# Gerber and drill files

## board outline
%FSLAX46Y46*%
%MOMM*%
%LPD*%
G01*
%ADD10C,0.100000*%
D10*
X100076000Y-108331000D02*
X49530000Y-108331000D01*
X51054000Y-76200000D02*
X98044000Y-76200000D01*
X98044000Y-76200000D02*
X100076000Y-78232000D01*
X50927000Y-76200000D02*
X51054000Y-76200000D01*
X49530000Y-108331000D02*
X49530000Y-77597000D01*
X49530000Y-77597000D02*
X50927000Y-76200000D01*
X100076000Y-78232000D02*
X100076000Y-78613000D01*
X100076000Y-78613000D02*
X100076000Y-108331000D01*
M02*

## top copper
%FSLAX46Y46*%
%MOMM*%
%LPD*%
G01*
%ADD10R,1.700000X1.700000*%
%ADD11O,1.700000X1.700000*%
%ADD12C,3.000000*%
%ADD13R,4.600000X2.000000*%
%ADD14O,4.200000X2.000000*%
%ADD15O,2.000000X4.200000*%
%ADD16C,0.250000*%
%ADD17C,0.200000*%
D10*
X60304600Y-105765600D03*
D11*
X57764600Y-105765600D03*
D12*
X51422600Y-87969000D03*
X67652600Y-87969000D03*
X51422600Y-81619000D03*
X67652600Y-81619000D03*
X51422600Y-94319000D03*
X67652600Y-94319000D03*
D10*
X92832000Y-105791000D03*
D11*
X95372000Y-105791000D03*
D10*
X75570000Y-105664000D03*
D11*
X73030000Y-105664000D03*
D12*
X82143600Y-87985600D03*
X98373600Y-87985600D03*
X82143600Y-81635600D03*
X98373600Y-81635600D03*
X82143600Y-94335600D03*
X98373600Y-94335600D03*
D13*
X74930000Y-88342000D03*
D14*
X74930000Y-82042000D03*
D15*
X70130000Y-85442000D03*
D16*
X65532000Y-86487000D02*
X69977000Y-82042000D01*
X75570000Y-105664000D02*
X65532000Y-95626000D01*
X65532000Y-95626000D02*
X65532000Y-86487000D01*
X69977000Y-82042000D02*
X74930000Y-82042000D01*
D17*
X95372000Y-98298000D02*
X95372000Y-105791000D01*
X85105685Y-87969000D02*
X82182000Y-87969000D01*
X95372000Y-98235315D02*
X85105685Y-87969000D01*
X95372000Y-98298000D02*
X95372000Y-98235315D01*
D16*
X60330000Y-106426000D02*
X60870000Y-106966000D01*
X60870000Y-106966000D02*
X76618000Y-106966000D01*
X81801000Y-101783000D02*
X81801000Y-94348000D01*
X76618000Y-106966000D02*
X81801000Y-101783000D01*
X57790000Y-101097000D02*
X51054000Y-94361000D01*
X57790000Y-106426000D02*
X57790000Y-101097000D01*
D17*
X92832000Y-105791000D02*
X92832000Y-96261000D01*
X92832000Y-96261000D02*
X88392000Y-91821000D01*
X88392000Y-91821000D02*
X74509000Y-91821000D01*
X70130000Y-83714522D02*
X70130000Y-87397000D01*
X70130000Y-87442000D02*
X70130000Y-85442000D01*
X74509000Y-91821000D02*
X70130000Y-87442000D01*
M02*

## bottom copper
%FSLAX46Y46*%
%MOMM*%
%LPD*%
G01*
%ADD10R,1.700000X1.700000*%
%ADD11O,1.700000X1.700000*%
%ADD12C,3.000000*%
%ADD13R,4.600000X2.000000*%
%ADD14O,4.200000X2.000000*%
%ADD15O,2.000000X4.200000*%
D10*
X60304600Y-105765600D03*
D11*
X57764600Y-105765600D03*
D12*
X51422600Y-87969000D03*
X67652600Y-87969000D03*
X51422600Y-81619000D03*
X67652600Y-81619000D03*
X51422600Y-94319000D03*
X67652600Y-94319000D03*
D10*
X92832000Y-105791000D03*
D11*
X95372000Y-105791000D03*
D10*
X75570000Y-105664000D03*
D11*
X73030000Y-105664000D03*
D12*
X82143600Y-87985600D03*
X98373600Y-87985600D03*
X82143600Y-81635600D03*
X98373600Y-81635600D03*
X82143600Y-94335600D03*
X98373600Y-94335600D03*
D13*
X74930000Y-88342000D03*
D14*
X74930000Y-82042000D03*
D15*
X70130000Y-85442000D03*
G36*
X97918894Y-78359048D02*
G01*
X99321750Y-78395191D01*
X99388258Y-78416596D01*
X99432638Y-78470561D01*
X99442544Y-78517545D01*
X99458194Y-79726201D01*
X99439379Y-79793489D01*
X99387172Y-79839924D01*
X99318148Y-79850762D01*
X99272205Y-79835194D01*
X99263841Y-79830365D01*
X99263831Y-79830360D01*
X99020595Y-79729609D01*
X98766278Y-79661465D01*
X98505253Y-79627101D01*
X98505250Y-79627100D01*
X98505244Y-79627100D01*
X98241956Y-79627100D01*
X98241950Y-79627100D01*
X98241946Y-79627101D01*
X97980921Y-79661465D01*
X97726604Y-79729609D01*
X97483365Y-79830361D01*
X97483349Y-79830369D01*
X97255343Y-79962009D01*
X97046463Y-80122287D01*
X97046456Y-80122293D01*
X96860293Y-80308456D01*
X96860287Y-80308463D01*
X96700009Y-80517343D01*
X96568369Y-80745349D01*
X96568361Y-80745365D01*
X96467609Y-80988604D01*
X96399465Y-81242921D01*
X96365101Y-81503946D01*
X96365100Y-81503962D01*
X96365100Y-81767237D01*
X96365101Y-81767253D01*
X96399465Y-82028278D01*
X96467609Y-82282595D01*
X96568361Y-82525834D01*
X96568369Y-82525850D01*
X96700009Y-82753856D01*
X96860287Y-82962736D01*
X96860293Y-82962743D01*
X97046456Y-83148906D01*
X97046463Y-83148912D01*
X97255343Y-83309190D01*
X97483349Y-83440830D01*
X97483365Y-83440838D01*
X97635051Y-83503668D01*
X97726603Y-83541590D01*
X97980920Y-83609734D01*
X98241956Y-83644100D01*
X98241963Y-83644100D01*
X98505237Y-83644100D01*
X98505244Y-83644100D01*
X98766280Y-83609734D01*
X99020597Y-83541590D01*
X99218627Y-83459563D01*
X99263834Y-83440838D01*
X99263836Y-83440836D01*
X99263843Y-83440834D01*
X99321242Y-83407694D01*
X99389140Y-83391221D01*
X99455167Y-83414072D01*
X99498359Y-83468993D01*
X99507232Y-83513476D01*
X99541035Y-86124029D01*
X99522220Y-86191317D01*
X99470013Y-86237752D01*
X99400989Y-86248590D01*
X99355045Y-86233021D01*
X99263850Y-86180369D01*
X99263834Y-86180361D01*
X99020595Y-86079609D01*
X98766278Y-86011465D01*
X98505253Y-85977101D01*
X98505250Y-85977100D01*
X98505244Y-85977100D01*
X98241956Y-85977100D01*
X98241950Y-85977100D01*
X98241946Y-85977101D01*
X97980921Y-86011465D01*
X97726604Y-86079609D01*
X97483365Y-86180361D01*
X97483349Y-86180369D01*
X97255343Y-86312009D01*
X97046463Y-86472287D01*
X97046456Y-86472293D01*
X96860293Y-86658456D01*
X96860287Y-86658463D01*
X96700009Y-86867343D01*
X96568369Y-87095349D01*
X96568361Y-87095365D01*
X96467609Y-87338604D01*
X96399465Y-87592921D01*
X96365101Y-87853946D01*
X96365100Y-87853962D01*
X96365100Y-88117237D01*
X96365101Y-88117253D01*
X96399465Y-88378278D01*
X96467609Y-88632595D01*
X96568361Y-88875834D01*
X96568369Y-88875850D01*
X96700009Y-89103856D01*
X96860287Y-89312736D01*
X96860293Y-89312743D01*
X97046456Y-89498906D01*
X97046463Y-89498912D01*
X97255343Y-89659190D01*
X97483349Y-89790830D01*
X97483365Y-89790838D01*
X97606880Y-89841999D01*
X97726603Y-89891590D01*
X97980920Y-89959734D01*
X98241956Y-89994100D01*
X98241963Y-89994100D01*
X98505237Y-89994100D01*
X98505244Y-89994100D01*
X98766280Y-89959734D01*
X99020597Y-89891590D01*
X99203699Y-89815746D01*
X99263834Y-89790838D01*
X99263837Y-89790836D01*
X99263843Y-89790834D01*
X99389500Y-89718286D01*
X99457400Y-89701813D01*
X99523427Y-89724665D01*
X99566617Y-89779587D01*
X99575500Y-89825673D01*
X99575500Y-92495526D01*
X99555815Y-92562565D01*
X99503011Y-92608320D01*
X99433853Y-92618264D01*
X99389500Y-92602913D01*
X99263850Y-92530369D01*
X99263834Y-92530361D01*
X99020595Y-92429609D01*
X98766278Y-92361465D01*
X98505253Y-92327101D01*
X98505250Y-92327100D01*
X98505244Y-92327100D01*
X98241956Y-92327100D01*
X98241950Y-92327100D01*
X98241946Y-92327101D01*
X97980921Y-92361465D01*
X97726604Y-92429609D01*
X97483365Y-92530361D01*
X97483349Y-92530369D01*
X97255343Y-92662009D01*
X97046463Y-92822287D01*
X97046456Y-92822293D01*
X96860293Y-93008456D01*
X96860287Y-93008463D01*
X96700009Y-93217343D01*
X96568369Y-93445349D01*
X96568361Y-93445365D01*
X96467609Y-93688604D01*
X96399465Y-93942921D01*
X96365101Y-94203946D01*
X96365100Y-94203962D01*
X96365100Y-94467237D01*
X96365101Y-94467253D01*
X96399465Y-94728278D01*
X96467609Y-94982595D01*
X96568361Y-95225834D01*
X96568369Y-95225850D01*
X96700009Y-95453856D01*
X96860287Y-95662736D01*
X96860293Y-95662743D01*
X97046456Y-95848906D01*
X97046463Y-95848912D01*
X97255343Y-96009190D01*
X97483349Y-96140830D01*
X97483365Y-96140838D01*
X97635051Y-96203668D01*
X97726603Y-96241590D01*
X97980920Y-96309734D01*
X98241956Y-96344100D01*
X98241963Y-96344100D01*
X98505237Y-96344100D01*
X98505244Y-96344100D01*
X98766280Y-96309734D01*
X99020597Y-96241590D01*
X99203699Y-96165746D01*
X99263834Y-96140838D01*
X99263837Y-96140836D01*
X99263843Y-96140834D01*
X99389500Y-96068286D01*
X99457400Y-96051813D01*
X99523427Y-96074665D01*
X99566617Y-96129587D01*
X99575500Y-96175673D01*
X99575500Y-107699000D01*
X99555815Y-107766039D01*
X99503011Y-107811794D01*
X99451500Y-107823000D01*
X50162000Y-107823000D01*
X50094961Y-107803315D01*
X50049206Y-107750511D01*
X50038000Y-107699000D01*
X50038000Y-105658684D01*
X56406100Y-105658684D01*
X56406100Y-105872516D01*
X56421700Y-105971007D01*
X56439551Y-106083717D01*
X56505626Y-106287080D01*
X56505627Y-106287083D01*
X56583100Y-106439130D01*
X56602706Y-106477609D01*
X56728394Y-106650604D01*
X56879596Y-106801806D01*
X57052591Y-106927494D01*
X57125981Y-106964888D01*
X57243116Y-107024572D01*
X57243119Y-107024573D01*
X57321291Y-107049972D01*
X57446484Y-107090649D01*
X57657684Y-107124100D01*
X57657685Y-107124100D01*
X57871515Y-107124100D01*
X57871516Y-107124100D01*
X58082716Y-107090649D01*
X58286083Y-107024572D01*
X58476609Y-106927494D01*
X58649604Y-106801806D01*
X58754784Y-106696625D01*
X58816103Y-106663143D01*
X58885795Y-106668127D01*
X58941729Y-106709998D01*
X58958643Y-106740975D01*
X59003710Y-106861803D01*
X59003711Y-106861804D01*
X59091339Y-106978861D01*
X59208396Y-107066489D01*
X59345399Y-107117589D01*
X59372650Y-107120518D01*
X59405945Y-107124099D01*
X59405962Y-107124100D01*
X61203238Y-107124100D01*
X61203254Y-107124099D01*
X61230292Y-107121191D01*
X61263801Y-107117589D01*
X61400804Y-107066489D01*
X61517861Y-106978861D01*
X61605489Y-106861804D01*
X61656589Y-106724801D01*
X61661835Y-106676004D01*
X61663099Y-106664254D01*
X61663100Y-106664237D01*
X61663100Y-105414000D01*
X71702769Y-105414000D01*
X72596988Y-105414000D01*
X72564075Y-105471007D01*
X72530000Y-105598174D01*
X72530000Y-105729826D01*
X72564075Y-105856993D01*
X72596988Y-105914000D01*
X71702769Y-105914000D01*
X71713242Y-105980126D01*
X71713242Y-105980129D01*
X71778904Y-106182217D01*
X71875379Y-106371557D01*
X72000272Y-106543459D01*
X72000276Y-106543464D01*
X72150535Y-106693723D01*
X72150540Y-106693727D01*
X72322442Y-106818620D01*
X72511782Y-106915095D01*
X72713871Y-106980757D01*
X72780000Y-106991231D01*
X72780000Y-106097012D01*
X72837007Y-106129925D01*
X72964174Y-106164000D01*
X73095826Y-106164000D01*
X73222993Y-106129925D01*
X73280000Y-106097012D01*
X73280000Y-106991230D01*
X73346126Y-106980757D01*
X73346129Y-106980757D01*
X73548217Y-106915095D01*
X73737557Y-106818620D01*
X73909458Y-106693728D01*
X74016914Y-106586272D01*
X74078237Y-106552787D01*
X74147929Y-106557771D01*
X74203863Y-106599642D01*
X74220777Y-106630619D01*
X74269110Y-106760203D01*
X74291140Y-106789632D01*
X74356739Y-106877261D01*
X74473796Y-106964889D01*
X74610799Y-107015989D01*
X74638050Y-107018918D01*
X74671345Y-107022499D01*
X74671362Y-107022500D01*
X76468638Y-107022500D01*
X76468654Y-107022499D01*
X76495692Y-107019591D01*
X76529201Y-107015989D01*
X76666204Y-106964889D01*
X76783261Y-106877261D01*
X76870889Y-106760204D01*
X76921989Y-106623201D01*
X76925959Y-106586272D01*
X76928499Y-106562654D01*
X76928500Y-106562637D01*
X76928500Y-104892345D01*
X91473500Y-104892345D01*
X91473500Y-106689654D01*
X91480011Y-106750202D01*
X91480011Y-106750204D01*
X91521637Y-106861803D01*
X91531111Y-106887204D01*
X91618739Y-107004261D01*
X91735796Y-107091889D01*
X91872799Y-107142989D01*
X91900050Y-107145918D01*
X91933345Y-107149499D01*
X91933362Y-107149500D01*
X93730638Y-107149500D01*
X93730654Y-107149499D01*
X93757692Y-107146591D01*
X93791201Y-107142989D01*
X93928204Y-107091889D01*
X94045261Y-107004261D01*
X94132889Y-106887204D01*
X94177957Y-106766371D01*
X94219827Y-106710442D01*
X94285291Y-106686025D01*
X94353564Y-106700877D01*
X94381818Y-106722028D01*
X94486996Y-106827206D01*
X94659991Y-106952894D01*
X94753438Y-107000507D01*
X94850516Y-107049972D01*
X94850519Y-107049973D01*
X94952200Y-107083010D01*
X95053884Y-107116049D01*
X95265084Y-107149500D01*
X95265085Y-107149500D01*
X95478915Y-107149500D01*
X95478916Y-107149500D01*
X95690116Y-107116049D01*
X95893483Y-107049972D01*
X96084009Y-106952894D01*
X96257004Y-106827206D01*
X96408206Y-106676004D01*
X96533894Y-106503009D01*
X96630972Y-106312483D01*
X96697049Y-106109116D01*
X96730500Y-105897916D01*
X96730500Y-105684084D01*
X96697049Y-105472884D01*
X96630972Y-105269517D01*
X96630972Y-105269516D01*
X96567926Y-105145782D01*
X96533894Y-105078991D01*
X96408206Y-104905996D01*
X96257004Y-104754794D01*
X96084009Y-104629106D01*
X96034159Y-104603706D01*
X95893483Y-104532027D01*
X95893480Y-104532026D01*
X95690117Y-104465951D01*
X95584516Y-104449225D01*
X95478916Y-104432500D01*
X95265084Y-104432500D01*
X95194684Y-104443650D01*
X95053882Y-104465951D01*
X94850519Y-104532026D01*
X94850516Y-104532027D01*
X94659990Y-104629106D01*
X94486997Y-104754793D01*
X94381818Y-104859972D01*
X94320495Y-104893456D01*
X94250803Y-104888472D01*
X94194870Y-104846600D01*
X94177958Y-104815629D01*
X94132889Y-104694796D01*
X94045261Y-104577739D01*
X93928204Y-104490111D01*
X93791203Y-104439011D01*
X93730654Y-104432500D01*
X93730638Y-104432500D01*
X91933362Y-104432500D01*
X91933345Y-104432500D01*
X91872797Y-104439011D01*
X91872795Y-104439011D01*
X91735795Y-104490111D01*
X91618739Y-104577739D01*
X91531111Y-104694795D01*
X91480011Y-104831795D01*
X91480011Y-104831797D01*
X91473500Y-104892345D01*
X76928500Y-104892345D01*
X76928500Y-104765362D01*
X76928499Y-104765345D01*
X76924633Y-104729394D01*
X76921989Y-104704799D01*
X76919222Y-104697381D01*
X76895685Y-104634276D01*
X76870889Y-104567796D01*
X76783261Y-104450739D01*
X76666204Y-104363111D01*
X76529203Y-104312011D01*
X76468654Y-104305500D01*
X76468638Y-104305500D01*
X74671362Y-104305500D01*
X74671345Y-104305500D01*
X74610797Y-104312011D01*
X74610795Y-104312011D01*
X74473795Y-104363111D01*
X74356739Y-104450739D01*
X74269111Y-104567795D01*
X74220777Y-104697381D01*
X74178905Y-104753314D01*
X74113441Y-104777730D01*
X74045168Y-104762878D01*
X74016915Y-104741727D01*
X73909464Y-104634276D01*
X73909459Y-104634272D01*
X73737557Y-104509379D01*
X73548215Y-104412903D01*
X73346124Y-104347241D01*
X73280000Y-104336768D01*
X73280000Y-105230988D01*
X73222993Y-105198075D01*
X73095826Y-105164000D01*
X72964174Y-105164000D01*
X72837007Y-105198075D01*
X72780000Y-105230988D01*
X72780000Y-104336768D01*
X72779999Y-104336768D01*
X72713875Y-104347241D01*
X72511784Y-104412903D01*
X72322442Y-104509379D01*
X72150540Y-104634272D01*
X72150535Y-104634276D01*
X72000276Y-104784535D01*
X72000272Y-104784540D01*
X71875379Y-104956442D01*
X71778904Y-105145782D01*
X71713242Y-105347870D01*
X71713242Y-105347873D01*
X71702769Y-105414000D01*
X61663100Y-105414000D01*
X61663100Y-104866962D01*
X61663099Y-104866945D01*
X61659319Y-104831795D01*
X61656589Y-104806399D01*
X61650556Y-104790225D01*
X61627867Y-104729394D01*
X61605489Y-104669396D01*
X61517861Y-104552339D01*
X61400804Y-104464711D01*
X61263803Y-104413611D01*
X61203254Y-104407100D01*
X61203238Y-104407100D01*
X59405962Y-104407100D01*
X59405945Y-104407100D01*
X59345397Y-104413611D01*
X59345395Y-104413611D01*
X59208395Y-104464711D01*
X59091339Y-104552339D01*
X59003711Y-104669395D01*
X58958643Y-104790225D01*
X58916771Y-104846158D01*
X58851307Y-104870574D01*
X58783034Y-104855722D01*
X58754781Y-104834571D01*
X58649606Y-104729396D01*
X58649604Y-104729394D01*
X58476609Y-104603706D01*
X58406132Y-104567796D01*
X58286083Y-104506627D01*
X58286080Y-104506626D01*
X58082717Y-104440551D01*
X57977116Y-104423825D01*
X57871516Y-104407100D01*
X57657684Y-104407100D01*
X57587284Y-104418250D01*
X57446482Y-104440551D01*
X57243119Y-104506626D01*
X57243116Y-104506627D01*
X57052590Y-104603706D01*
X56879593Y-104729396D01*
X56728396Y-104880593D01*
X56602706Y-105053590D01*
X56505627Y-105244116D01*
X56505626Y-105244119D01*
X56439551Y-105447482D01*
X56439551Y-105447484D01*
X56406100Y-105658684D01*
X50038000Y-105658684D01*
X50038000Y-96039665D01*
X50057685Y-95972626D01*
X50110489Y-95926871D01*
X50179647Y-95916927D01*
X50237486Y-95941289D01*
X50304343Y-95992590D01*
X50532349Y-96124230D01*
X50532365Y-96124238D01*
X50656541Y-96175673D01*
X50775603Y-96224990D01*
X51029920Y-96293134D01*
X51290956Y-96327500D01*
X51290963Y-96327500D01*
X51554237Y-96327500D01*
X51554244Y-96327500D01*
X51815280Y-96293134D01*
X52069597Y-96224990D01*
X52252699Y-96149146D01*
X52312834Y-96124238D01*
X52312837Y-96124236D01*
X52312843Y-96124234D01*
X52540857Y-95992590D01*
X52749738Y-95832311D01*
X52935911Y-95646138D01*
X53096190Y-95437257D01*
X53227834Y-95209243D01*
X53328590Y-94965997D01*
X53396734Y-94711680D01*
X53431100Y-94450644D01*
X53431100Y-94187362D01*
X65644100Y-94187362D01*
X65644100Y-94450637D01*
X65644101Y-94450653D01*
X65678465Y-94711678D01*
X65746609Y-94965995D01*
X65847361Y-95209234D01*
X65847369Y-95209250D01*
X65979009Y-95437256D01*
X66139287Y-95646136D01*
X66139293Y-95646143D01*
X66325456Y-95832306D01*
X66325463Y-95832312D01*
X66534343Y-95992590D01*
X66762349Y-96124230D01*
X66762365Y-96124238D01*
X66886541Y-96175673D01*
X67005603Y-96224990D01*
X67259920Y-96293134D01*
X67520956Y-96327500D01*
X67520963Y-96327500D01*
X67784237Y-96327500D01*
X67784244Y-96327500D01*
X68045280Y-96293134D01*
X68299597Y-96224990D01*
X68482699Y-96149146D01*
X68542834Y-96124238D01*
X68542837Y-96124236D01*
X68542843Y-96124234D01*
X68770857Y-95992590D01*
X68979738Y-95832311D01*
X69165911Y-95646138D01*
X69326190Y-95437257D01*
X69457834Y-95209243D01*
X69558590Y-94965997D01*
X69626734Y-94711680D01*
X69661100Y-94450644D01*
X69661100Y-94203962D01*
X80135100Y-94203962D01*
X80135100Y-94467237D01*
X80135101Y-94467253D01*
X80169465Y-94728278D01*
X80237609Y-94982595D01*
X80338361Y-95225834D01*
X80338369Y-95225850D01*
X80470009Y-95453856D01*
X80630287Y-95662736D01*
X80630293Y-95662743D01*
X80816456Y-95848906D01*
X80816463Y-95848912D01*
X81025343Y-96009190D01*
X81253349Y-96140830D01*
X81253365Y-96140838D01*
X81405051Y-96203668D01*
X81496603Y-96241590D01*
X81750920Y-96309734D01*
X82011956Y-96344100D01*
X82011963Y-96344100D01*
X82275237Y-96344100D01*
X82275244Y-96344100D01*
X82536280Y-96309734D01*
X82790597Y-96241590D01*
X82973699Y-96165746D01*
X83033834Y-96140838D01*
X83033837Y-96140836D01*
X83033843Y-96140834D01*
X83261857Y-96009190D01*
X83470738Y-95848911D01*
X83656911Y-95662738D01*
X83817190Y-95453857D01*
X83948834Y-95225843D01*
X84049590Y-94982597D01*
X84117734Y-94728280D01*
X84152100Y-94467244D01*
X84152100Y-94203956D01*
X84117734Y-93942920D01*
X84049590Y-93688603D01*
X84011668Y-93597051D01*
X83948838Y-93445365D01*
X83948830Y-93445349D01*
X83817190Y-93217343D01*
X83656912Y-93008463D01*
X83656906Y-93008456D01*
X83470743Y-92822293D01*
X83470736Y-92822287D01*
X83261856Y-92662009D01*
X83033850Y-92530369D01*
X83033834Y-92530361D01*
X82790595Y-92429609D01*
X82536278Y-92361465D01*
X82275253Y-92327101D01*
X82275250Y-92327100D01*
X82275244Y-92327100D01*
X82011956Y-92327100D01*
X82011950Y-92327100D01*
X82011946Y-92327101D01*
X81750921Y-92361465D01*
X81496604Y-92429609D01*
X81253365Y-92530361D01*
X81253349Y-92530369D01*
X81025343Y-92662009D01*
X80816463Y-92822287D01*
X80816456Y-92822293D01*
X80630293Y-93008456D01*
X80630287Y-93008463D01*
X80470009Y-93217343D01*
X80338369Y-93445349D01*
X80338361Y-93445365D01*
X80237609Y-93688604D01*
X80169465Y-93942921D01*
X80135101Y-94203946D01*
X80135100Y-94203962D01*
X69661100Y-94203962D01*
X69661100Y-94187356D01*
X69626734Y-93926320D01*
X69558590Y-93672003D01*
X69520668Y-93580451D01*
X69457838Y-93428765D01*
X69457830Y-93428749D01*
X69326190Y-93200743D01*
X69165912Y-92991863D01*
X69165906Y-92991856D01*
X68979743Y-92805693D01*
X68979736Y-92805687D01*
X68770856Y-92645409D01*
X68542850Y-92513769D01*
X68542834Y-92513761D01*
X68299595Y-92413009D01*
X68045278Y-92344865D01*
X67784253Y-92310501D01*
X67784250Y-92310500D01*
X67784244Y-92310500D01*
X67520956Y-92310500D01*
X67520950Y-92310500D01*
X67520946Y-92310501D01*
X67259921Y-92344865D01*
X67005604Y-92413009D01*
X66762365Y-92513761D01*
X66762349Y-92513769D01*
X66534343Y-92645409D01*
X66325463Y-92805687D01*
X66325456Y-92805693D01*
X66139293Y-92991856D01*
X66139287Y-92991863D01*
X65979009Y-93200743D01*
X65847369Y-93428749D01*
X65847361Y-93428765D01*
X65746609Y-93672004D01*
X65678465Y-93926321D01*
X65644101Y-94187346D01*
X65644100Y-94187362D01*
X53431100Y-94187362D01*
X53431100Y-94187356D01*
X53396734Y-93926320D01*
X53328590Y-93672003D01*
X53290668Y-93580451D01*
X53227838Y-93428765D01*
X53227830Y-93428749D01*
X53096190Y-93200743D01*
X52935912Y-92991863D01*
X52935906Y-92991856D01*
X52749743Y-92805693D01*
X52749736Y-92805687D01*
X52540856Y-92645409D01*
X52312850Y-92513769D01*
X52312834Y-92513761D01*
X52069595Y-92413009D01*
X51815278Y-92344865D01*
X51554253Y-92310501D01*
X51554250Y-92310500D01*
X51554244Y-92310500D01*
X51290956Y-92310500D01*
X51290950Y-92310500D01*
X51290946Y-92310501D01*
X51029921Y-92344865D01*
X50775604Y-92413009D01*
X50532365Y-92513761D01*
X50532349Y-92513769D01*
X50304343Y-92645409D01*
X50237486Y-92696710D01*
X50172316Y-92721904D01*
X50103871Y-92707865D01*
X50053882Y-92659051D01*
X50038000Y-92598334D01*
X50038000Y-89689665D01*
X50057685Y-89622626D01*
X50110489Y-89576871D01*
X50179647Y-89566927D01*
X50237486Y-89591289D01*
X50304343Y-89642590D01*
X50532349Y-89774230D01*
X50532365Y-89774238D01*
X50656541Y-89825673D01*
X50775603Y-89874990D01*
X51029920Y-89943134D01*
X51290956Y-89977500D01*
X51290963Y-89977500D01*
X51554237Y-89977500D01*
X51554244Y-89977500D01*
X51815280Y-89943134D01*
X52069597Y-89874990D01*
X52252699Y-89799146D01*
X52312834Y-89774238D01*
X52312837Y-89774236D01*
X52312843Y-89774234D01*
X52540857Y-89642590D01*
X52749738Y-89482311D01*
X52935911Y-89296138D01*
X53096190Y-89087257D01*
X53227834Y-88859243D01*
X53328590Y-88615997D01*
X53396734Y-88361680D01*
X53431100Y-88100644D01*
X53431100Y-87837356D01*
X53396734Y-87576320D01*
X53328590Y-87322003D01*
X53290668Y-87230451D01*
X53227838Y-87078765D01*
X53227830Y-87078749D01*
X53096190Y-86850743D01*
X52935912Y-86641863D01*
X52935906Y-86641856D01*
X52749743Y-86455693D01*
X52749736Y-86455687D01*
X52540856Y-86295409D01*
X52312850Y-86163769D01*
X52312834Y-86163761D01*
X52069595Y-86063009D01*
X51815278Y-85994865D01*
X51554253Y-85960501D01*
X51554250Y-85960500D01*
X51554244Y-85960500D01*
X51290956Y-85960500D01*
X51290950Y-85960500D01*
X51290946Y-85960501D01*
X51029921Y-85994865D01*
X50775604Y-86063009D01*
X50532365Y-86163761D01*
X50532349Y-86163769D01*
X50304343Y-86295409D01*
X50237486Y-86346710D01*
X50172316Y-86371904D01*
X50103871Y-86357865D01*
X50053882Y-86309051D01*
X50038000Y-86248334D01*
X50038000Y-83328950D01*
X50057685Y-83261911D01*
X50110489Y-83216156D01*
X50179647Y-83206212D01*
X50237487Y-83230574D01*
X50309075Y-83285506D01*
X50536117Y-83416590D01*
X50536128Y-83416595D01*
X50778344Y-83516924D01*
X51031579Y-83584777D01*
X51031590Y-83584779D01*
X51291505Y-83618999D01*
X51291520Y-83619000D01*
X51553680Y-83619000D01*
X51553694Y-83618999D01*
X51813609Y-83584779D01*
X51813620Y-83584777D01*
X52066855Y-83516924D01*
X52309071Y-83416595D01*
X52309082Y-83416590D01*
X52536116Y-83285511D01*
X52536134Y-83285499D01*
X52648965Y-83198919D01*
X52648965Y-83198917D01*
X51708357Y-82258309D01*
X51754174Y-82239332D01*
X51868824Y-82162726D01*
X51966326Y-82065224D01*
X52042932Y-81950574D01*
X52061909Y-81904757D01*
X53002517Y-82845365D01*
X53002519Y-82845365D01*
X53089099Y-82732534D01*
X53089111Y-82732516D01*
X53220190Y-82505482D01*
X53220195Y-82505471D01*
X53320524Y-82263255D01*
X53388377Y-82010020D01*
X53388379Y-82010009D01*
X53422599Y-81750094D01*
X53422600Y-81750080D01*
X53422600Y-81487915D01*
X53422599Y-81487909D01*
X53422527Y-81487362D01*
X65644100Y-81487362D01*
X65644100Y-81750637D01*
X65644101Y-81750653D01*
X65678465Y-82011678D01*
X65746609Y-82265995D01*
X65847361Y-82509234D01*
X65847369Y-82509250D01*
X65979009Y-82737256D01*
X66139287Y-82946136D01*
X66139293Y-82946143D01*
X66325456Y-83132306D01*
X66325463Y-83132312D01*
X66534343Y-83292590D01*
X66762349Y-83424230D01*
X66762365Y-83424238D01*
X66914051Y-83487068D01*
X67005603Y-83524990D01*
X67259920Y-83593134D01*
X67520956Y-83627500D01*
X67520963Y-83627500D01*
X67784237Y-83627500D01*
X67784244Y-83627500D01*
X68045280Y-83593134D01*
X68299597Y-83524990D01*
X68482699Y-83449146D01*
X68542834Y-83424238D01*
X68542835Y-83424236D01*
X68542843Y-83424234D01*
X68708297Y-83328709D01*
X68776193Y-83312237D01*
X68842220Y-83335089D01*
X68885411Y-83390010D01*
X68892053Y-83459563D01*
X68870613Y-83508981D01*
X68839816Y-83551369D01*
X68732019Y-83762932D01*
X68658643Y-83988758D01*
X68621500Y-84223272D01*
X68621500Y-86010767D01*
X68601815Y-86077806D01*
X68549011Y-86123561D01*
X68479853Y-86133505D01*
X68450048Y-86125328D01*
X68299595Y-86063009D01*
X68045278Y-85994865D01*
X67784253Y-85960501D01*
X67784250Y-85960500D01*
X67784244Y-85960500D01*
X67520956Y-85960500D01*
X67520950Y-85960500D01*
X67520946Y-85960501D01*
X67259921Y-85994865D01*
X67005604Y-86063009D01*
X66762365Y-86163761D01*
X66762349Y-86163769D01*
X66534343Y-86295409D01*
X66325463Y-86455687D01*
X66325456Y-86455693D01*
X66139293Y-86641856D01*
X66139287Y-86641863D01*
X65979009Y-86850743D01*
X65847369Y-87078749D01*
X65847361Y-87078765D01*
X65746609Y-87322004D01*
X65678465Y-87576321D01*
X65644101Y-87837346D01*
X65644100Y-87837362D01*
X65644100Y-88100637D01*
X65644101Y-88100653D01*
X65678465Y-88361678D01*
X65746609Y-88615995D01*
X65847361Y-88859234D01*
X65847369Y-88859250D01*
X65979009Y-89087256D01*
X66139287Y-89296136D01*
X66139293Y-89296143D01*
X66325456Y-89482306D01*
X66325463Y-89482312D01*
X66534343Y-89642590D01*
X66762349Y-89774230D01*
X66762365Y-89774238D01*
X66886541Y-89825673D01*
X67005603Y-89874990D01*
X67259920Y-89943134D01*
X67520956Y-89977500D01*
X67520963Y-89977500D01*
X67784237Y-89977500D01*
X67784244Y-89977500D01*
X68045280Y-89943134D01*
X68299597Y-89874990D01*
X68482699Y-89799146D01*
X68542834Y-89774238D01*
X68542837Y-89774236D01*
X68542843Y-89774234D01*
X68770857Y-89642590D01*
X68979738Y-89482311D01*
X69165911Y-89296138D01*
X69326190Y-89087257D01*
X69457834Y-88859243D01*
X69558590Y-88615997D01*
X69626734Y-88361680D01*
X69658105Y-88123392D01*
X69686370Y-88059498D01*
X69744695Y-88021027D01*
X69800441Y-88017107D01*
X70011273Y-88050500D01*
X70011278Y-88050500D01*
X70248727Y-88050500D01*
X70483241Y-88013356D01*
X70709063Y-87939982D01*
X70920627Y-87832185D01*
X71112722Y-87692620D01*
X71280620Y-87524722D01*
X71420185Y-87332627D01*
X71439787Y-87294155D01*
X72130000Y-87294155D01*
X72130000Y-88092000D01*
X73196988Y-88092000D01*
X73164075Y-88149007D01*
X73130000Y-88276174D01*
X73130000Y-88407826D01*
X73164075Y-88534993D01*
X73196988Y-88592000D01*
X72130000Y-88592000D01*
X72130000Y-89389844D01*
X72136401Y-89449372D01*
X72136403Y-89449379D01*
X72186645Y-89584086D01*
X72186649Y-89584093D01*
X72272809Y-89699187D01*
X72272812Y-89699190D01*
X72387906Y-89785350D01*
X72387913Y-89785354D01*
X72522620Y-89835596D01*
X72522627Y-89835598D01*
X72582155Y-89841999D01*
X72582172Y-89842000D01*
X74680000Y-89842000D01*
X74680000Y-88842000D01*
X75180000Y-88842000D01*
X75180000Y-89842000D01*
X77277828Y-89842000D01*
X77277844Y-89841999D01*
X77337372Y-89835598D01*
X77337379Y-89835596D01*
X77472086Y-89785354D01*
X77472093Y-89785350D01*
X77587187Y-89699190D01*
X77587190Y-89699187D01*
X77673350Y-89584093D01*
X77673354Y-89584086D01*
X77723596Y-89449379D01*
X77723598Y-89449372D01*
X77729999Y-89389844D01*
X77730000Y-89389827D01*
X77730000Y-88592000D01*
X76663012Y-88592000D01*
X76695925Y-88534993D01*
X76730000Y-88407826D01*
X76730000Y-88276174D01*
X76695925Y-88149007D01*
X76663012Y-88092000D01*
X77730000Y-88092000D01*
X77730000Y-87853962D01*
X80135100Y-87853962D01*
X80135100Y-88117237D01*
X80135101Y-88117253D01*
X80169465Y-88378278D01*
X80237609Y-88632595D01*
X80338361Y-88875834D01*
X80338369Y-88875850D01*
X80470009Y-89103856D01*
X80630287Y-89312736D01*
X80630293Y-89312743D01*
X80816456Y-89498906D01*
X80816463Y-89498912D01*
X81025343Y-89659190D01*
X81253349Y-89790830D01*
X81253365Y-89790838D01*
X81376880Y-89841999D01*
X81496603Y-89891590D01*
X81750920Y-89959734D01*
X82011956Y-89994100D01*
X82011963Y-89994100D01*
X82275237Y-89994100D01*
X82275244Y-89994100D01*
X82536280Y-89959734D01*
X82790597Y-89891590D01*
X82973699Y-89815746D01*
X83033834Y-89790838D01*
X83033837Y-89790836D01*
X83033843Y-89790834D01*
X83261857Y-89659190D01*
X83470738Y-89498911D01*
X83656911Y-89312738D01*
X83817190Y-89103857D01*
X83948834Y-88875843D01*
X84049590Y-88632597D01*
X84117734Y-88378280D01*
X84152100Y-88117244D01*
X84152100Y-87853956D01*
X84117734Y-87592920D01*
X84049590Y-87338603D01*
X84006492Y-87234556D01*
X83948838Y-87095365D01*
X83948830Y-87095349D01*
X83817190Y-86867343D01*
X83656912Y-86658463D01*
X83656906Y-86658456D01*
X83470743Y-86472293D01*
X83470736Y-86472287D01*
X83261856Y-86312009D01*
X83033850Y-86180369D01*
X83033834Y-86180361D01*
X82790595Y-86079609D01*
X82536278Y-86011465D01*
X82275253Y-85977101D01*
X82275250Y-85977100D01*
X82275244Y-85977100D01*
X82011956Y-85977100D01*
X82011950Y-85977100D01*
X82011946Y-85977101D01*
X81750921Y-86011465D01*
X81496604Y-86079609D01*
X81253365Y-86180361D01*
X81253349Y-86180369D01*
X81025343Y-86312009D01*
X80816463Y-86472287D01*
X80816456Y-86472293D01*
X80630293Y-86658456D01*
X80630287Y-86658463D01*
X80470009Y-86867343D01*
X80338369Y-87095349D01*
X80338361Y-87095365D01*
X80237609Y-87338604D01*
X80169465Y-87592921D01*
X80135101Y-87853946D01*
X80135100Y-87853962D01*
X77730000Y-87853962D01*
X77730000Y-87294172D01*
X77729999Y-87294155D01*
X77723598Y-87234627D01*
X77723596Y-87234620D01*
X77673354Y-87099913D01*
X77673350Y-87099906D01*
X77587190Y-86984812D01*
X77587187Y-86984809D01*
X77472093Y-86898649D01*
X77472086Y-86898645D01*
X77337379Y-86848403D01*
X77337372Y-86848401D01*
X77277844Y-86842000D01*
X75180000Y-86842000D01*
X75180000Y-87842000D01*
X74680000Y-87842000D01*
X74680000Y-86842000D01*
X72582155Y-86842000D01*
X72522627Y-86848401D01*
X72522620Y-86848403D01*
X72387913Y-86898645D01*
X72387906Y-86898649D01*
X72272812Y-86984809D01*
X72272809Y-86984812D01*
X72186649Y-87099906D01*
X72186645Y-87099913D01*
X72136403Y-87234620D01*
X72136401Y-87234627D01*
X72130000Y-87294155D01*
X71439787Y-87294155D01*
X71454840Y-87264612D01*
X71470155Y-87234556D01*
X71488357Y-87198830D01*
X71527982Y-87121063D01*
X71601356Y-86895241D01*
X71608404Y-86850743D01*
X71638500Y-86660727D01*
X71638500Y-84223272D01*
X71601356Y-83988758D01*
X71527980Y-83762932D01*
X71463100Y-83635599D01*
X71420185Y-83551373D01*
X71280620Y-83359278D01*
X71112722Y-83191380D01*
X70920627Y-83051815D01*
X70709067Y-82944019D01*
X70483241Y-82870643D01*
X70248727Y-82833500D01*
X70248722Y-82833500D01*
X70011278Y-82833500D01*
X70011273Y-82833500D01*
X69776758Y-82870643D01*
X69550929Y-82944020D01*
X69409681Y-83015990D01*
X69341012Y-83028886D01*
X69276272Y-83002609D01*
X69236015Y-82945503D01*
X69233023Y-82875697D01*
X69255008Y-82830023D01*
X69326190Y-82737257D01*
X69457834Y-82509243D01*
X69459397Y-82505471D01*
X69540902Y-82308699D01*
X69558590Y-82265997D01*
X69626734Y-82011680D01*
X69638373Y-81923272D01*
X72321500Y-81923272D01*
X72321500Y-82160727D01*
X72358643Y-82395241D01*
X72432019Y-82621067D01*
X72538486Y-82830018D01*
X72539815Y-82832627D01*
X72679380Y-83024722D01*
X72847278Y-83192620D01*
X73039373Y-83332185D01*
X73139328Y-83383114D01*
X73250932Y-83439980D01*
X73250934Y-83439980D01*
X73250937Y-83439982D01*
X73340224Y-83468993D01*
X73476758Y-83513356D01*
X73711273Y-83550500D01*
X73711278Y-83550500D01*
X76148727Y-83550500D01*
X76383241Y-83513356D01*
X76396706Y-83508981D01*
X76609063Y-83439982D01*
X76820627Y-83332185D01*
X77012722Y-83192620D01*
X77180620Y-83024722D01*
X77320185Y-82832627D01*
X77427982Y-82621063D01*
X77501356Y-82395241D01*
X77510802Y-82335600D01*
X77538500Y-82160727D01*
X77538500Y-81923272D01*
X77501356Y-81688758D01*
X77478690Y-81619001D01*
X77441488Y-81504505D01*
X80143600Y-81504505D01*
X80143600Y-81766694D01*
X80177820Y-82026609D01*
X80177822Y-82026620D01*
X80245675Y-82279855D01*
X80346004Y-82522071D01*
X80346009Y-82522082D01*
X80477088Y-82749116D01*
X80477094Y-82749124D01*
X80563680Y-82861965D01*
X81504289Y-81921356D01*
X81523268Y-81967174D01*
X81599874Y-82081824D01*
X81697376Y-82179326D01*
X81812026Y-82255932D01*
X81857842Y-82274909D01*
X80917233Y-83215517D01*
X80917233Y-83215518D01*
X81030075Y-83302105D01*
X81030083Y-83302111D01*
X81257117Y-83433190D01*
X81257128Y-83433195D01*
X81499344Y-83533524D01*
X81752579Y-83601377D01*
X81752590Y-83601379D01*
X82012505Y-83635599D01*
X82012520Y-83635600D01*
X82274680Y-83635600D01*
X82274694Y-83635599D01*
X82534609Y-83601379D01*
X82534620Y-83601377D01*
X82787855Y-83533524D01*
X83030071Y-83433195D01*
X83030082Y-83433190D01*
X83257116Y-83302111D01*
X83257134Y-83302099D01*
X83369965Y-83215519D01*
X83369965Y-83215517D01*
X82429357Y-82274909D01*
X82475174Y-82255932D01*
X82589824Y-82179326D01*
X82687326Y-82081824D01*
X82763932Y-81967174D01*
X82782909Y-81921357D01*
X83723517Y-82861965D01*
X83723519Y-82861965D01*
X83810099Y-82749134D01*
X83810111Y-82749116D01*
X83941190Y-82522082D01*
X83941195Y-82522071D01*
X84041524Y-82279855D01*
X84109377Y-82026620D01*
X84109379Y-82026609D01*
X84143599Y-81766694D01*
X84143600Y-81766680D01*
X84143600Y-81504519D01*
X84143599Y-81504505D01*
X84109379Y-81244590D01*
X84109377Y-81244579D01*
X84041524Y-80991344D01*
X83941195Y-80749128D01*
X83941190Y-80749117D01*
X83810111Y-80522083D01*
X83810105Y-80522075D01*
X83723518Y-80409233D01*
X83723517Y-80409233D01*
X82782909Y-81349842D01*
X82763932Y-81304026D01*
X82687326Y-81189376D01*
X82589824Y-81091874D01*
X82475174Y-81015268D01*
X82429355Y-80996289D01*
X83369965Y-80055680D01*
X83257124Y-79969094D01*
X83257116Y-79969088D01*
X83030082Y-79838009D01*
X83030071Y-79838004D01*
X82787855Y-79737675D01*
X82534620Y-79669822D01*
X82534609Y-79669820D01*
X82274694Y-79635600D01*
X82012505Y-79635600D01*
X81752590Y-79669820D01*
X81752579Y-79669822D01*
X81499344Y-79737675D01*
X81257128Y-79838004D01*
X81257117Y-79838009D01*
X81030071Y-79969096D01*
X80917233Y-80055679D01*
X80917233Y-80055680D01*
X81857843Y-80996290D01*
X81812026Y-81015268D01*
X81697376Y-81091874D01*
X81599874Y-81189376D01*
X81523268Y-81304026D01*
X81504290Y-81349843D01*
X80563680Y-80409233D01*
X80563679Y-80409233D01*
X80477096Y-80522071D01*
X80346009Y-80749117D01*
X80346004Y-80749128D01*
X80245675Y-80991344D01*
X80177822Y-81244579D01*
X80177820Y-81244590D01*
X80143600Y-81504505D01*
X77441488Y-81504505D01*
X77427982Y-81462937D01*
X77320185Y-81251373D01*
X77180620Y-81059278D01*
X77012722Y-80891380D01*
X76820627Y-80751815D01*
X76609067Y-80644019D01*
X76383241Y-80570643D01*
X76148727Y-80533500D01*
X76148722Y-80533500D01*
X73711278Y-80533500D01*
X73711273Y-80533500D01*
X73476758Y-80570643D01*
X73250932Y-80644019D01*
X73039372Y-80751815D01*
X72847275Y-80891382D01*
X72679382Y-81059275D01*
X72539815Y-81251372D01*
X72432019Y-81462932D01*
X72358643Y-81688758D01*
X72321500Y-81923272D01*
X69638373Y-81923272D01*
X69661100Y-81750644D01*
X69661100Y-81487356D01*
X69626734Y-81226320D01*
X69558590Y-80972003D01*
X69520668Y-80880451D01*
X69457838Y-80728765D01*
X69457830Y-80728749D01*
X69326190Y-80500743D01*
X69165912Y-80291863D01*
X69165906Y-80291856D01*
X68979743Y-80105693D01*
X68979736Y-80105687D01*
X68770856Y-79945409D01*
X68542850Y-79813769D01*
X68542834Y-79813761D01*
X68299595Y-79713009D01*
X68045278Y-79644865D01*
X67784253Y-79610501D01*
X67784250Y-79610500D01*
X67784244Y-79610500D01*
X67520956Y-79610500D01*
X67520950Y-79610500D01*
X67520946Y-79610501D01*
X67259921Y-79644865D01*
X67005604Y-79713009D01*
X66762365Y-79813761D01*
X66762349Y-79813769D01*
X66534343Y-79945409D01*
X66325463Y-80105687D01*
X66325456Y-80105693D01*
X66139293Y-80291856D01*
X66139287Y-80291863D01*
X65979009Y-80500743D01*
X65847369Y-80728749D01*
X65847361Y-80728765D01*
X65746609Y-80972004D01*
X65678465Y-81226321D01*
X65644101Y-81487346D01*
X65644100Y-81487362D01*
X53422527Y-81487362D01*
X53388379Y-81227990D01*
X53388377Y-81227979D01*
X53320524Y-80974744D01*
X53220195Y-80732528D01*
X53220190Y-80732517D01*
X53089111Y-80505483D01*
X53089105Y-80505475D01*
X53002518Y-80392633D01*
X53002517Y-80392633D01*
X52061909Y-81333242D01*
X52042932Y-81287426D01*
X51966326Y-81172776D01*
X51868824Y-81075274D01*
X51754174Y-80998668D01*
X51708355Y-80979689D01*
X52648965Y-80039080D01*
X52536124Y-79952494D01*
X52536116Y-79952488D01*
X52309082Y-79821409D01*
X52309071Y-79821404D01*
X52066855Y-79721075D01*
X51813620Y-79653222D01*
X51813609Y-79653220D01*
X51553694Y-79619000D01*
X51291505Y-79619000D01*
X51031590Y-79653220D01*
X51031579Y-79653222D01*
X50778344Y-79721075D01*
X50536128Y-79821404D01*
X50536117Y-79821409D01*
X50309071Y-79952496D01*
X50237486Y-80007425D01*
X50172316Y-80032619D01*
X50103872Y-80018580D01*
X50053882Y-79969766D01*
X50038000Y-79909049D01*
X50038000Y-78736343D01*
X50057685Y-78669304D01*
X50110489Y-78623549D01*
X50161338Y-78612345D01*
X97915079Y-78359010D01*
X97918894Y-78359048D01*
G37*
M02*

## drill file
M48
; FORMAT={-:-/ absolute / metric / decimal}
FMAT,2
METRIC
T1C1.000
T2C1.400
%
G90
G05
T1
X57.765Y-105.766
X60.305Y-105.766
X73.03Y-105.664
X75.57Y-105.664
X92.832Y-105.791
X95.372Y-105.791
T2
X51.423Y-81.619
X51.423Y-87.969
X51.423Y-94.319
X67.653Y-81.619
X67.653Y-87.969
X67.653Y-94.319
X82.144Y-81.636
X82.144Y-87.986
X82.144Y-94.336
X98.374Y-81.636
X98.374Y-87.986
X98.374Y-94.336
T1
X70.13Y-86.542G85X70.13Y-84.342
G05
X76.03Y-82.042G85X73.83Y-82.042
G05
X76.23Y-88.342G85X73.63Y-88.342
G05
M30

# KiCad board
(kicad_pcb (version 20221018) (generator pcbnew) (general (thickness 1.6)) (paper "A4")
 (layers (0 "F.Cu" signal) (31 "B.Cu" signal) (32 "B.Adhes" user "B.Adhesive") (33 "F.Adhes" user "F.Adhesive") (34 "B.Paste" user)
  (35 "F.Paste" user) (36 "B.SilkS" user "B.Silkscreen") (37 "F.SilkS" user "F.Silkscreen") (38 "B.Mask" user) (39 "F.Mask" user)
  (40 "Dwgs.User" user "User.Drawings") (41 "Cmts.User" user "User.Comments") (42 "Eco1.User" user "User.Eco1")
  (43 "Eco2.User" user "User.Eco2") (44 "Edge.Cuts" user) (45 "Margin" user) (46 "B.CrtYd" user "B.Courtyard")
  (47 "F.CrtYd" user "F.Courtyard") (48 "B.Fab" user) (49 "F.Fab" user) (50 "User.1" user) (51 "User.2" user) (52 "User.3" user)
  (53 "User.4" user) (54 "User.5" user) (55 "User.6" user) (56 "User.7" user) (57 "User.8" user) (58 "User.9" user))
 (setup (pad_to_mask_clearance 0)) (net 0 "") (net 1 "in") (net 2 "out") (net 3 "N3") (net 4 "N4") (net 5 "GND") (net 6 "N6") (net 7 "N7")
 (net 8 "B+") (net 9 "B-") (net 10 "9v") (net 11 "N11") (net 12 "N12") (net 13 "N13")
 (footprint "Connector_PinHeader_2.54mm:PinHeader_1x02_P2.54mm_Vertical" (layer "F.Cu") (at 60.3046 105.7656 -90)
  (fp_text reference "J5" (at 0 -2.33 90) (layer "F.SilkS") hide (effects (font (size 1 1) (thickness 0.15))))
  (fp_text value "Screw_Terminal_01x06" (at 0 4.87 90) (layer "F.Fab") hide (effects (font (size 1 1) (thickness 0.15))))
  (pad "1" thru_hole rect (at 0 0 270) (size 1.7 1.7) (drill 1) (layers "*.Cu" "*.Mask") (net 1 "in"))
  (pad "2" thru_hole oval (at 0 2.54 270) (size 1.7 1.7) (drill 1) (layers "*.Cu" "*.Mask") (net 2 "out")))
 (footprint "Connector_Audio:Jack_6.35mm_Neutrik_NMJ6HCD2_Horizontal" (layer "F.Cu") (at 51.4226 94.319 90)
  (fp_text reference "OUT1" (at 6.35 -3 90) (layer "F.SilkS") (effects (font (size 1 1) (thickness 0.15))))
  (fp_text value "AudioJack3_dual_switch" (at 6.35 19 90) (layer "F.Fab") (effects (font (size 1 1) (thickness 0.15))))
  (pad "R" thru_hole circle (at 6.35 0 90) (size 3 3) (drill 1.4) (layers "*.Cu" "*.Mask") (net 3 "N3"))
  (pad "RN" thru_hole circle (at 6.35 16.23 90) (size 3 3) (drill 1.4) (layers "*.Cu" "*.Mask") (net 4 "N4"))
  (pad "S" thru_hole circle (at 12.7 0 90) (size 3 3) (drill 1.4) (layers "*.Cu" "*.Mask") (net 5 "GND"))
  (pad "SN" thru_hole circle (at 12.7 16.23 90) (size 3 3) (drill 1.4) (layers "*.Cu" "*.Mask") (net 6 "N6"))
  (pad "T" thru_hole circle (at 0 0 90) (size 3 3) (drill 1.4) (layers "*.Cu" "*.Mask") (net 2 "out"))
  (pad "TN" thru_hole circle (at 0 16.23 90) (size 3 3) (drill 1.4) (layers "*.Cu" "*.Mask") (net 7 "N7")))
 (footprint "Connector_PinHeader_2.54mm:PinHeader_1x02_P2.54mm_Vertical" (layer "F.Cu") (at 92.832 105.791 90)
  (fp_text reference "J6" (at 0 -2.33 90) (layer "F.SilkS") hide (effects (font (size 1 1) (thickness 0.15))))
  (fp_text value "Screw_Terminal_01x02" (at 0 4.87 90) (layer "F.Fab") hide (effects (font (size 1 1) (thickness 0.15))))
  (pad "1" thru_hole rect (at 0 0 90) (size 1.7 1.7) (drill 1) (layers "*.Cu" "*.Mask") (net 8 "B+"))
  (pad "2" thru_hole oval (at 0 2.54 90) (size 1.7 1.7) (drill 1) (layers "*.Cu" "*.Mask") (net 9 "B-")))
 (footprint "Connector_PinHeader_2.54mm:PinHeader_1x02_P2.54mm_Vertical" (layer "F.Cu") (at 75.57 105.664 -90)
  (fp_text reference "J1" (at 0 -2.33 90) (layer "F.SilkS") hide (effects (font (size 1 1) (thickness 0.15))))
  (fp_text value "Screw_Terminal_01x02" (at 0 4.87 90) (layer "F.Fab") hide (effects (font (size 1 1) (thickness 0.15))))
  (pad "1" thru_hole rect (at 0 0 270) (size 1.7 1.7) (drill 1) (layers "*.Cu" "*.Mask") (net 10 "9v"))
  (pad "2" thru_hole oval (at 0 2.54 270) (size 1.7 1.7) (drill 1) (layers "*.Cu" "*.Mask") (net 5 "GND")))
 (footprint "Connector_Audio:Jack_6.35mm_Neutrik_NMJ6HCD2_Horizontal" (layer "F.Cu") (at 82.1436 94.3356 90)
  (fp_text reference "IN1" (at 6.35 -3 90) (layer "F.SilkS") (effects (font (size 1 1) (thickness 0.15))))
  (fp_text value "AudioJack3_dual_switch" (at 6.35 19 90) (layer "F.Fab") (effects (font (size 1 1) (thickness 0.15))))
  (pad "R" thru_hole circle (at 6.35 0 90) (size 3 3) (drill 1.4) (layers "*.Cu" "*.Mask") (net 9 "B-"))
  (pad "RN" thru_hole circle (at 6.35 16.23 90) (size 3 3) (drill 1.4) (layers "*.Cu" "*.Mask") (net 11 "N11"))
  (pad "S" thru_hole circle (at 12.7 0 90) (size 3 3) (drill 1.4) (layers "*.Cu" "*.Mask") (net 5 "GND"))
  (pad "SN" thru_hole circle (at 12.7 16.23 90) (size 3 3) (drill 1.4) (layers "*.Cu" "*.Mask") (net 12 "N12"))
  (pad "T" thru_hole circle (at 0 0 90) (size 3 3) (drill 1.4) (layers "*.Cu" "*.Mask") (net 1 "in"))
  (pad "TN" thru_hole circle (at 0 16.23 90) (size 3 3) (drill 1.4) (layers "*.Cu" "*.Mask") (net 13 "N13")))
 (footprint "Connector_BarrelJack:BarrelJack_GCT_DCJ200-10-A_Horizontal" (layer "F.Cu") (at 74.93 88.342 180)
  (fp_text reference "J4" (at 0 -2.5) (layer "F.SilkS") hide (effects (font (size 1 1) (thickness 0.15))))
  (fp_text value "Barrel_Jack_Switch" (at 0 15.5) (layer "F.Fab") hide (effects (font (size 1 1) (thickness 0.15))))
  (pad "1" thru_hole rect (at 0 0 180) (size 4.6 2) (drill oval 3.6 1) (layers "*.Cu" "*.Mask") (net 5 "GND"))
  (pad "2" thru_hole oval (at 0 6.3 180) (size 4.2 2) (drill oval 3.2 1) (layers "*.Cu" "*.Mask") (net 10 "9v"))
  (pad "3" thru_hole oval (at 4.8 2.9 180) (size 2 4.2) (drill oval 1 3.2) (layers "*.Cu" "*.Mask") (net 8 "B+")))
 (gr_line (start 100.076 108.331) (end 49.53 108.331) (stroke (width 0.1) (type default)) (layer "Edge.Cuts"))
 (gr_line (start 51.054 76.2) (end 98.044 76.2) (stroke (width 0.1) (type default)) (layer "Edge.Cuts"))
 (gr_line (start 98.044 76.2) (end 100.076 78.232) (stroke (width 0.1) (type default)) (layer "Edge.Cuts"))
 (gr_line (start 50.927 76.2) (end 51.054 76.2) (stroke (width 0.1) (type default)) (layer "Edge.Cuts"))
 (gr_line (start 49.53 108.331) (end 49.53 77.597) (stroke (width 0.1) (type default)) (layer "Edge.Cuts"))
 (gr_line (start 49.53 77.597) (end 50.927 76.2) (stroke (width 0.1) (type default)) (layer "Edge.Cuts"))
 (gr_line (start 100.076 78.232) (end 100.076 78.613) (stroke (width 0.1) (type default)) (layer "Edge.Cuts"))
 (gr_line (start 100.076 78.613) (end 100.076 108.331) (stroke (width 0.1) (type default)) (layer "Edge.Cuts"))
 (segment (start 65.532 86.487) (end 69.977 82.042) (width 0.25) (layer "F.Cu") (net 10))
 (segment (start 75.57 105.664) (end 65.532 95.626) (width 0.25) (layer "F.Cu") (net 10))
 (segment (start 65.532 95.626) (end 65.532 86.487) (width 0.25) (layer "F.Cu") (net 10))
 (segment (start 69.977 82.042) (end 74.93 82.042) (width 0.25) (layer "F.Cu") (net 10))
 (segment (start 95.372 98.298) (end 95.372 105.791) (width 0.2) (layer "F.Cu") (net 9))
 (segment (start 85.105685 87.969) (end 82.182 87.969) (width 0.2) (layer "F.Cu") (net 9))
 (segment (start 95.372 98.235315) (end 85.105685 87.969) (width 0.2) (layer "F.Cu") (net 9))
 (segment (start 95.372 98.298) (end 95.372 98.235315) (width 0.2) (layer "F.Cu") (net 9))
 (segment (start 60.33 106.426) (end 60.87 106.966) (width 0.25) (layer "F.Cu") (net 1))
 (segment (start 60.87 106.966) (end 76.618 106.966) (width 0.25) (layer "F.Cu") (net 1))
 (segment (start 81.801 101.783) (end 81.801 94.348) (width 0.25) (layer "F.Cu") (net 1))
 (segment (start 76.618 106.966) (end 81.801 101.783) (width 0.25) (layer "F.Cu") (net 1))
 (segment (start 57.79 101.097) (end 51.054 94.361) (width 0.25) (layer "F.Cu") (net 2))
 (segment (start 57.79 106.426) (end 57.79 101.097) (width 0.25) (layer "F.Cu") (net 2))
 (segment (start 92.832 105.791) (end 92.832 96.261) (width 0.2) (layer "F.Cu") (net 8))
 (segment (start 92.832 96.261) (end 88.392 91.821) (width 0.2) (layer "F.Cu") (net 8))
 (segment (start 88.392 91.821) (end 74.509 91.821) (width 0.2) (layer "F.Cu") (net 8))
 (segment (start 70.13 83.714522) (end 70.13 87.397) (width 0.2) (layer "F.Cu") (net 8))
 (segment (start 70.13 87.442) (end 70.13 85.442) (width 0.2) (layer "F.Cu") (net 8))
 (segment (start 74.509 91.821) (end 70.13 87.442) (width 0.2) (layer "F.Cu") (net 8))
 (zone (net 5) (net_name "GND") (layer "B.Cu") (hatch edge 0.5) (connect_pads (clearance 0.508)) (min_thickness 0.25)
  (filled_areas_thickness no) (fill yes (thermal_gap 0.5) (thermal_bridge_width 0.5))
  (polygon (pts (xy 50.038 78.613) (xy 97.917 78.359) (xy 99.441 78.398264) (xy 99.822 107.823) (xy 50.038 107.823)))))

